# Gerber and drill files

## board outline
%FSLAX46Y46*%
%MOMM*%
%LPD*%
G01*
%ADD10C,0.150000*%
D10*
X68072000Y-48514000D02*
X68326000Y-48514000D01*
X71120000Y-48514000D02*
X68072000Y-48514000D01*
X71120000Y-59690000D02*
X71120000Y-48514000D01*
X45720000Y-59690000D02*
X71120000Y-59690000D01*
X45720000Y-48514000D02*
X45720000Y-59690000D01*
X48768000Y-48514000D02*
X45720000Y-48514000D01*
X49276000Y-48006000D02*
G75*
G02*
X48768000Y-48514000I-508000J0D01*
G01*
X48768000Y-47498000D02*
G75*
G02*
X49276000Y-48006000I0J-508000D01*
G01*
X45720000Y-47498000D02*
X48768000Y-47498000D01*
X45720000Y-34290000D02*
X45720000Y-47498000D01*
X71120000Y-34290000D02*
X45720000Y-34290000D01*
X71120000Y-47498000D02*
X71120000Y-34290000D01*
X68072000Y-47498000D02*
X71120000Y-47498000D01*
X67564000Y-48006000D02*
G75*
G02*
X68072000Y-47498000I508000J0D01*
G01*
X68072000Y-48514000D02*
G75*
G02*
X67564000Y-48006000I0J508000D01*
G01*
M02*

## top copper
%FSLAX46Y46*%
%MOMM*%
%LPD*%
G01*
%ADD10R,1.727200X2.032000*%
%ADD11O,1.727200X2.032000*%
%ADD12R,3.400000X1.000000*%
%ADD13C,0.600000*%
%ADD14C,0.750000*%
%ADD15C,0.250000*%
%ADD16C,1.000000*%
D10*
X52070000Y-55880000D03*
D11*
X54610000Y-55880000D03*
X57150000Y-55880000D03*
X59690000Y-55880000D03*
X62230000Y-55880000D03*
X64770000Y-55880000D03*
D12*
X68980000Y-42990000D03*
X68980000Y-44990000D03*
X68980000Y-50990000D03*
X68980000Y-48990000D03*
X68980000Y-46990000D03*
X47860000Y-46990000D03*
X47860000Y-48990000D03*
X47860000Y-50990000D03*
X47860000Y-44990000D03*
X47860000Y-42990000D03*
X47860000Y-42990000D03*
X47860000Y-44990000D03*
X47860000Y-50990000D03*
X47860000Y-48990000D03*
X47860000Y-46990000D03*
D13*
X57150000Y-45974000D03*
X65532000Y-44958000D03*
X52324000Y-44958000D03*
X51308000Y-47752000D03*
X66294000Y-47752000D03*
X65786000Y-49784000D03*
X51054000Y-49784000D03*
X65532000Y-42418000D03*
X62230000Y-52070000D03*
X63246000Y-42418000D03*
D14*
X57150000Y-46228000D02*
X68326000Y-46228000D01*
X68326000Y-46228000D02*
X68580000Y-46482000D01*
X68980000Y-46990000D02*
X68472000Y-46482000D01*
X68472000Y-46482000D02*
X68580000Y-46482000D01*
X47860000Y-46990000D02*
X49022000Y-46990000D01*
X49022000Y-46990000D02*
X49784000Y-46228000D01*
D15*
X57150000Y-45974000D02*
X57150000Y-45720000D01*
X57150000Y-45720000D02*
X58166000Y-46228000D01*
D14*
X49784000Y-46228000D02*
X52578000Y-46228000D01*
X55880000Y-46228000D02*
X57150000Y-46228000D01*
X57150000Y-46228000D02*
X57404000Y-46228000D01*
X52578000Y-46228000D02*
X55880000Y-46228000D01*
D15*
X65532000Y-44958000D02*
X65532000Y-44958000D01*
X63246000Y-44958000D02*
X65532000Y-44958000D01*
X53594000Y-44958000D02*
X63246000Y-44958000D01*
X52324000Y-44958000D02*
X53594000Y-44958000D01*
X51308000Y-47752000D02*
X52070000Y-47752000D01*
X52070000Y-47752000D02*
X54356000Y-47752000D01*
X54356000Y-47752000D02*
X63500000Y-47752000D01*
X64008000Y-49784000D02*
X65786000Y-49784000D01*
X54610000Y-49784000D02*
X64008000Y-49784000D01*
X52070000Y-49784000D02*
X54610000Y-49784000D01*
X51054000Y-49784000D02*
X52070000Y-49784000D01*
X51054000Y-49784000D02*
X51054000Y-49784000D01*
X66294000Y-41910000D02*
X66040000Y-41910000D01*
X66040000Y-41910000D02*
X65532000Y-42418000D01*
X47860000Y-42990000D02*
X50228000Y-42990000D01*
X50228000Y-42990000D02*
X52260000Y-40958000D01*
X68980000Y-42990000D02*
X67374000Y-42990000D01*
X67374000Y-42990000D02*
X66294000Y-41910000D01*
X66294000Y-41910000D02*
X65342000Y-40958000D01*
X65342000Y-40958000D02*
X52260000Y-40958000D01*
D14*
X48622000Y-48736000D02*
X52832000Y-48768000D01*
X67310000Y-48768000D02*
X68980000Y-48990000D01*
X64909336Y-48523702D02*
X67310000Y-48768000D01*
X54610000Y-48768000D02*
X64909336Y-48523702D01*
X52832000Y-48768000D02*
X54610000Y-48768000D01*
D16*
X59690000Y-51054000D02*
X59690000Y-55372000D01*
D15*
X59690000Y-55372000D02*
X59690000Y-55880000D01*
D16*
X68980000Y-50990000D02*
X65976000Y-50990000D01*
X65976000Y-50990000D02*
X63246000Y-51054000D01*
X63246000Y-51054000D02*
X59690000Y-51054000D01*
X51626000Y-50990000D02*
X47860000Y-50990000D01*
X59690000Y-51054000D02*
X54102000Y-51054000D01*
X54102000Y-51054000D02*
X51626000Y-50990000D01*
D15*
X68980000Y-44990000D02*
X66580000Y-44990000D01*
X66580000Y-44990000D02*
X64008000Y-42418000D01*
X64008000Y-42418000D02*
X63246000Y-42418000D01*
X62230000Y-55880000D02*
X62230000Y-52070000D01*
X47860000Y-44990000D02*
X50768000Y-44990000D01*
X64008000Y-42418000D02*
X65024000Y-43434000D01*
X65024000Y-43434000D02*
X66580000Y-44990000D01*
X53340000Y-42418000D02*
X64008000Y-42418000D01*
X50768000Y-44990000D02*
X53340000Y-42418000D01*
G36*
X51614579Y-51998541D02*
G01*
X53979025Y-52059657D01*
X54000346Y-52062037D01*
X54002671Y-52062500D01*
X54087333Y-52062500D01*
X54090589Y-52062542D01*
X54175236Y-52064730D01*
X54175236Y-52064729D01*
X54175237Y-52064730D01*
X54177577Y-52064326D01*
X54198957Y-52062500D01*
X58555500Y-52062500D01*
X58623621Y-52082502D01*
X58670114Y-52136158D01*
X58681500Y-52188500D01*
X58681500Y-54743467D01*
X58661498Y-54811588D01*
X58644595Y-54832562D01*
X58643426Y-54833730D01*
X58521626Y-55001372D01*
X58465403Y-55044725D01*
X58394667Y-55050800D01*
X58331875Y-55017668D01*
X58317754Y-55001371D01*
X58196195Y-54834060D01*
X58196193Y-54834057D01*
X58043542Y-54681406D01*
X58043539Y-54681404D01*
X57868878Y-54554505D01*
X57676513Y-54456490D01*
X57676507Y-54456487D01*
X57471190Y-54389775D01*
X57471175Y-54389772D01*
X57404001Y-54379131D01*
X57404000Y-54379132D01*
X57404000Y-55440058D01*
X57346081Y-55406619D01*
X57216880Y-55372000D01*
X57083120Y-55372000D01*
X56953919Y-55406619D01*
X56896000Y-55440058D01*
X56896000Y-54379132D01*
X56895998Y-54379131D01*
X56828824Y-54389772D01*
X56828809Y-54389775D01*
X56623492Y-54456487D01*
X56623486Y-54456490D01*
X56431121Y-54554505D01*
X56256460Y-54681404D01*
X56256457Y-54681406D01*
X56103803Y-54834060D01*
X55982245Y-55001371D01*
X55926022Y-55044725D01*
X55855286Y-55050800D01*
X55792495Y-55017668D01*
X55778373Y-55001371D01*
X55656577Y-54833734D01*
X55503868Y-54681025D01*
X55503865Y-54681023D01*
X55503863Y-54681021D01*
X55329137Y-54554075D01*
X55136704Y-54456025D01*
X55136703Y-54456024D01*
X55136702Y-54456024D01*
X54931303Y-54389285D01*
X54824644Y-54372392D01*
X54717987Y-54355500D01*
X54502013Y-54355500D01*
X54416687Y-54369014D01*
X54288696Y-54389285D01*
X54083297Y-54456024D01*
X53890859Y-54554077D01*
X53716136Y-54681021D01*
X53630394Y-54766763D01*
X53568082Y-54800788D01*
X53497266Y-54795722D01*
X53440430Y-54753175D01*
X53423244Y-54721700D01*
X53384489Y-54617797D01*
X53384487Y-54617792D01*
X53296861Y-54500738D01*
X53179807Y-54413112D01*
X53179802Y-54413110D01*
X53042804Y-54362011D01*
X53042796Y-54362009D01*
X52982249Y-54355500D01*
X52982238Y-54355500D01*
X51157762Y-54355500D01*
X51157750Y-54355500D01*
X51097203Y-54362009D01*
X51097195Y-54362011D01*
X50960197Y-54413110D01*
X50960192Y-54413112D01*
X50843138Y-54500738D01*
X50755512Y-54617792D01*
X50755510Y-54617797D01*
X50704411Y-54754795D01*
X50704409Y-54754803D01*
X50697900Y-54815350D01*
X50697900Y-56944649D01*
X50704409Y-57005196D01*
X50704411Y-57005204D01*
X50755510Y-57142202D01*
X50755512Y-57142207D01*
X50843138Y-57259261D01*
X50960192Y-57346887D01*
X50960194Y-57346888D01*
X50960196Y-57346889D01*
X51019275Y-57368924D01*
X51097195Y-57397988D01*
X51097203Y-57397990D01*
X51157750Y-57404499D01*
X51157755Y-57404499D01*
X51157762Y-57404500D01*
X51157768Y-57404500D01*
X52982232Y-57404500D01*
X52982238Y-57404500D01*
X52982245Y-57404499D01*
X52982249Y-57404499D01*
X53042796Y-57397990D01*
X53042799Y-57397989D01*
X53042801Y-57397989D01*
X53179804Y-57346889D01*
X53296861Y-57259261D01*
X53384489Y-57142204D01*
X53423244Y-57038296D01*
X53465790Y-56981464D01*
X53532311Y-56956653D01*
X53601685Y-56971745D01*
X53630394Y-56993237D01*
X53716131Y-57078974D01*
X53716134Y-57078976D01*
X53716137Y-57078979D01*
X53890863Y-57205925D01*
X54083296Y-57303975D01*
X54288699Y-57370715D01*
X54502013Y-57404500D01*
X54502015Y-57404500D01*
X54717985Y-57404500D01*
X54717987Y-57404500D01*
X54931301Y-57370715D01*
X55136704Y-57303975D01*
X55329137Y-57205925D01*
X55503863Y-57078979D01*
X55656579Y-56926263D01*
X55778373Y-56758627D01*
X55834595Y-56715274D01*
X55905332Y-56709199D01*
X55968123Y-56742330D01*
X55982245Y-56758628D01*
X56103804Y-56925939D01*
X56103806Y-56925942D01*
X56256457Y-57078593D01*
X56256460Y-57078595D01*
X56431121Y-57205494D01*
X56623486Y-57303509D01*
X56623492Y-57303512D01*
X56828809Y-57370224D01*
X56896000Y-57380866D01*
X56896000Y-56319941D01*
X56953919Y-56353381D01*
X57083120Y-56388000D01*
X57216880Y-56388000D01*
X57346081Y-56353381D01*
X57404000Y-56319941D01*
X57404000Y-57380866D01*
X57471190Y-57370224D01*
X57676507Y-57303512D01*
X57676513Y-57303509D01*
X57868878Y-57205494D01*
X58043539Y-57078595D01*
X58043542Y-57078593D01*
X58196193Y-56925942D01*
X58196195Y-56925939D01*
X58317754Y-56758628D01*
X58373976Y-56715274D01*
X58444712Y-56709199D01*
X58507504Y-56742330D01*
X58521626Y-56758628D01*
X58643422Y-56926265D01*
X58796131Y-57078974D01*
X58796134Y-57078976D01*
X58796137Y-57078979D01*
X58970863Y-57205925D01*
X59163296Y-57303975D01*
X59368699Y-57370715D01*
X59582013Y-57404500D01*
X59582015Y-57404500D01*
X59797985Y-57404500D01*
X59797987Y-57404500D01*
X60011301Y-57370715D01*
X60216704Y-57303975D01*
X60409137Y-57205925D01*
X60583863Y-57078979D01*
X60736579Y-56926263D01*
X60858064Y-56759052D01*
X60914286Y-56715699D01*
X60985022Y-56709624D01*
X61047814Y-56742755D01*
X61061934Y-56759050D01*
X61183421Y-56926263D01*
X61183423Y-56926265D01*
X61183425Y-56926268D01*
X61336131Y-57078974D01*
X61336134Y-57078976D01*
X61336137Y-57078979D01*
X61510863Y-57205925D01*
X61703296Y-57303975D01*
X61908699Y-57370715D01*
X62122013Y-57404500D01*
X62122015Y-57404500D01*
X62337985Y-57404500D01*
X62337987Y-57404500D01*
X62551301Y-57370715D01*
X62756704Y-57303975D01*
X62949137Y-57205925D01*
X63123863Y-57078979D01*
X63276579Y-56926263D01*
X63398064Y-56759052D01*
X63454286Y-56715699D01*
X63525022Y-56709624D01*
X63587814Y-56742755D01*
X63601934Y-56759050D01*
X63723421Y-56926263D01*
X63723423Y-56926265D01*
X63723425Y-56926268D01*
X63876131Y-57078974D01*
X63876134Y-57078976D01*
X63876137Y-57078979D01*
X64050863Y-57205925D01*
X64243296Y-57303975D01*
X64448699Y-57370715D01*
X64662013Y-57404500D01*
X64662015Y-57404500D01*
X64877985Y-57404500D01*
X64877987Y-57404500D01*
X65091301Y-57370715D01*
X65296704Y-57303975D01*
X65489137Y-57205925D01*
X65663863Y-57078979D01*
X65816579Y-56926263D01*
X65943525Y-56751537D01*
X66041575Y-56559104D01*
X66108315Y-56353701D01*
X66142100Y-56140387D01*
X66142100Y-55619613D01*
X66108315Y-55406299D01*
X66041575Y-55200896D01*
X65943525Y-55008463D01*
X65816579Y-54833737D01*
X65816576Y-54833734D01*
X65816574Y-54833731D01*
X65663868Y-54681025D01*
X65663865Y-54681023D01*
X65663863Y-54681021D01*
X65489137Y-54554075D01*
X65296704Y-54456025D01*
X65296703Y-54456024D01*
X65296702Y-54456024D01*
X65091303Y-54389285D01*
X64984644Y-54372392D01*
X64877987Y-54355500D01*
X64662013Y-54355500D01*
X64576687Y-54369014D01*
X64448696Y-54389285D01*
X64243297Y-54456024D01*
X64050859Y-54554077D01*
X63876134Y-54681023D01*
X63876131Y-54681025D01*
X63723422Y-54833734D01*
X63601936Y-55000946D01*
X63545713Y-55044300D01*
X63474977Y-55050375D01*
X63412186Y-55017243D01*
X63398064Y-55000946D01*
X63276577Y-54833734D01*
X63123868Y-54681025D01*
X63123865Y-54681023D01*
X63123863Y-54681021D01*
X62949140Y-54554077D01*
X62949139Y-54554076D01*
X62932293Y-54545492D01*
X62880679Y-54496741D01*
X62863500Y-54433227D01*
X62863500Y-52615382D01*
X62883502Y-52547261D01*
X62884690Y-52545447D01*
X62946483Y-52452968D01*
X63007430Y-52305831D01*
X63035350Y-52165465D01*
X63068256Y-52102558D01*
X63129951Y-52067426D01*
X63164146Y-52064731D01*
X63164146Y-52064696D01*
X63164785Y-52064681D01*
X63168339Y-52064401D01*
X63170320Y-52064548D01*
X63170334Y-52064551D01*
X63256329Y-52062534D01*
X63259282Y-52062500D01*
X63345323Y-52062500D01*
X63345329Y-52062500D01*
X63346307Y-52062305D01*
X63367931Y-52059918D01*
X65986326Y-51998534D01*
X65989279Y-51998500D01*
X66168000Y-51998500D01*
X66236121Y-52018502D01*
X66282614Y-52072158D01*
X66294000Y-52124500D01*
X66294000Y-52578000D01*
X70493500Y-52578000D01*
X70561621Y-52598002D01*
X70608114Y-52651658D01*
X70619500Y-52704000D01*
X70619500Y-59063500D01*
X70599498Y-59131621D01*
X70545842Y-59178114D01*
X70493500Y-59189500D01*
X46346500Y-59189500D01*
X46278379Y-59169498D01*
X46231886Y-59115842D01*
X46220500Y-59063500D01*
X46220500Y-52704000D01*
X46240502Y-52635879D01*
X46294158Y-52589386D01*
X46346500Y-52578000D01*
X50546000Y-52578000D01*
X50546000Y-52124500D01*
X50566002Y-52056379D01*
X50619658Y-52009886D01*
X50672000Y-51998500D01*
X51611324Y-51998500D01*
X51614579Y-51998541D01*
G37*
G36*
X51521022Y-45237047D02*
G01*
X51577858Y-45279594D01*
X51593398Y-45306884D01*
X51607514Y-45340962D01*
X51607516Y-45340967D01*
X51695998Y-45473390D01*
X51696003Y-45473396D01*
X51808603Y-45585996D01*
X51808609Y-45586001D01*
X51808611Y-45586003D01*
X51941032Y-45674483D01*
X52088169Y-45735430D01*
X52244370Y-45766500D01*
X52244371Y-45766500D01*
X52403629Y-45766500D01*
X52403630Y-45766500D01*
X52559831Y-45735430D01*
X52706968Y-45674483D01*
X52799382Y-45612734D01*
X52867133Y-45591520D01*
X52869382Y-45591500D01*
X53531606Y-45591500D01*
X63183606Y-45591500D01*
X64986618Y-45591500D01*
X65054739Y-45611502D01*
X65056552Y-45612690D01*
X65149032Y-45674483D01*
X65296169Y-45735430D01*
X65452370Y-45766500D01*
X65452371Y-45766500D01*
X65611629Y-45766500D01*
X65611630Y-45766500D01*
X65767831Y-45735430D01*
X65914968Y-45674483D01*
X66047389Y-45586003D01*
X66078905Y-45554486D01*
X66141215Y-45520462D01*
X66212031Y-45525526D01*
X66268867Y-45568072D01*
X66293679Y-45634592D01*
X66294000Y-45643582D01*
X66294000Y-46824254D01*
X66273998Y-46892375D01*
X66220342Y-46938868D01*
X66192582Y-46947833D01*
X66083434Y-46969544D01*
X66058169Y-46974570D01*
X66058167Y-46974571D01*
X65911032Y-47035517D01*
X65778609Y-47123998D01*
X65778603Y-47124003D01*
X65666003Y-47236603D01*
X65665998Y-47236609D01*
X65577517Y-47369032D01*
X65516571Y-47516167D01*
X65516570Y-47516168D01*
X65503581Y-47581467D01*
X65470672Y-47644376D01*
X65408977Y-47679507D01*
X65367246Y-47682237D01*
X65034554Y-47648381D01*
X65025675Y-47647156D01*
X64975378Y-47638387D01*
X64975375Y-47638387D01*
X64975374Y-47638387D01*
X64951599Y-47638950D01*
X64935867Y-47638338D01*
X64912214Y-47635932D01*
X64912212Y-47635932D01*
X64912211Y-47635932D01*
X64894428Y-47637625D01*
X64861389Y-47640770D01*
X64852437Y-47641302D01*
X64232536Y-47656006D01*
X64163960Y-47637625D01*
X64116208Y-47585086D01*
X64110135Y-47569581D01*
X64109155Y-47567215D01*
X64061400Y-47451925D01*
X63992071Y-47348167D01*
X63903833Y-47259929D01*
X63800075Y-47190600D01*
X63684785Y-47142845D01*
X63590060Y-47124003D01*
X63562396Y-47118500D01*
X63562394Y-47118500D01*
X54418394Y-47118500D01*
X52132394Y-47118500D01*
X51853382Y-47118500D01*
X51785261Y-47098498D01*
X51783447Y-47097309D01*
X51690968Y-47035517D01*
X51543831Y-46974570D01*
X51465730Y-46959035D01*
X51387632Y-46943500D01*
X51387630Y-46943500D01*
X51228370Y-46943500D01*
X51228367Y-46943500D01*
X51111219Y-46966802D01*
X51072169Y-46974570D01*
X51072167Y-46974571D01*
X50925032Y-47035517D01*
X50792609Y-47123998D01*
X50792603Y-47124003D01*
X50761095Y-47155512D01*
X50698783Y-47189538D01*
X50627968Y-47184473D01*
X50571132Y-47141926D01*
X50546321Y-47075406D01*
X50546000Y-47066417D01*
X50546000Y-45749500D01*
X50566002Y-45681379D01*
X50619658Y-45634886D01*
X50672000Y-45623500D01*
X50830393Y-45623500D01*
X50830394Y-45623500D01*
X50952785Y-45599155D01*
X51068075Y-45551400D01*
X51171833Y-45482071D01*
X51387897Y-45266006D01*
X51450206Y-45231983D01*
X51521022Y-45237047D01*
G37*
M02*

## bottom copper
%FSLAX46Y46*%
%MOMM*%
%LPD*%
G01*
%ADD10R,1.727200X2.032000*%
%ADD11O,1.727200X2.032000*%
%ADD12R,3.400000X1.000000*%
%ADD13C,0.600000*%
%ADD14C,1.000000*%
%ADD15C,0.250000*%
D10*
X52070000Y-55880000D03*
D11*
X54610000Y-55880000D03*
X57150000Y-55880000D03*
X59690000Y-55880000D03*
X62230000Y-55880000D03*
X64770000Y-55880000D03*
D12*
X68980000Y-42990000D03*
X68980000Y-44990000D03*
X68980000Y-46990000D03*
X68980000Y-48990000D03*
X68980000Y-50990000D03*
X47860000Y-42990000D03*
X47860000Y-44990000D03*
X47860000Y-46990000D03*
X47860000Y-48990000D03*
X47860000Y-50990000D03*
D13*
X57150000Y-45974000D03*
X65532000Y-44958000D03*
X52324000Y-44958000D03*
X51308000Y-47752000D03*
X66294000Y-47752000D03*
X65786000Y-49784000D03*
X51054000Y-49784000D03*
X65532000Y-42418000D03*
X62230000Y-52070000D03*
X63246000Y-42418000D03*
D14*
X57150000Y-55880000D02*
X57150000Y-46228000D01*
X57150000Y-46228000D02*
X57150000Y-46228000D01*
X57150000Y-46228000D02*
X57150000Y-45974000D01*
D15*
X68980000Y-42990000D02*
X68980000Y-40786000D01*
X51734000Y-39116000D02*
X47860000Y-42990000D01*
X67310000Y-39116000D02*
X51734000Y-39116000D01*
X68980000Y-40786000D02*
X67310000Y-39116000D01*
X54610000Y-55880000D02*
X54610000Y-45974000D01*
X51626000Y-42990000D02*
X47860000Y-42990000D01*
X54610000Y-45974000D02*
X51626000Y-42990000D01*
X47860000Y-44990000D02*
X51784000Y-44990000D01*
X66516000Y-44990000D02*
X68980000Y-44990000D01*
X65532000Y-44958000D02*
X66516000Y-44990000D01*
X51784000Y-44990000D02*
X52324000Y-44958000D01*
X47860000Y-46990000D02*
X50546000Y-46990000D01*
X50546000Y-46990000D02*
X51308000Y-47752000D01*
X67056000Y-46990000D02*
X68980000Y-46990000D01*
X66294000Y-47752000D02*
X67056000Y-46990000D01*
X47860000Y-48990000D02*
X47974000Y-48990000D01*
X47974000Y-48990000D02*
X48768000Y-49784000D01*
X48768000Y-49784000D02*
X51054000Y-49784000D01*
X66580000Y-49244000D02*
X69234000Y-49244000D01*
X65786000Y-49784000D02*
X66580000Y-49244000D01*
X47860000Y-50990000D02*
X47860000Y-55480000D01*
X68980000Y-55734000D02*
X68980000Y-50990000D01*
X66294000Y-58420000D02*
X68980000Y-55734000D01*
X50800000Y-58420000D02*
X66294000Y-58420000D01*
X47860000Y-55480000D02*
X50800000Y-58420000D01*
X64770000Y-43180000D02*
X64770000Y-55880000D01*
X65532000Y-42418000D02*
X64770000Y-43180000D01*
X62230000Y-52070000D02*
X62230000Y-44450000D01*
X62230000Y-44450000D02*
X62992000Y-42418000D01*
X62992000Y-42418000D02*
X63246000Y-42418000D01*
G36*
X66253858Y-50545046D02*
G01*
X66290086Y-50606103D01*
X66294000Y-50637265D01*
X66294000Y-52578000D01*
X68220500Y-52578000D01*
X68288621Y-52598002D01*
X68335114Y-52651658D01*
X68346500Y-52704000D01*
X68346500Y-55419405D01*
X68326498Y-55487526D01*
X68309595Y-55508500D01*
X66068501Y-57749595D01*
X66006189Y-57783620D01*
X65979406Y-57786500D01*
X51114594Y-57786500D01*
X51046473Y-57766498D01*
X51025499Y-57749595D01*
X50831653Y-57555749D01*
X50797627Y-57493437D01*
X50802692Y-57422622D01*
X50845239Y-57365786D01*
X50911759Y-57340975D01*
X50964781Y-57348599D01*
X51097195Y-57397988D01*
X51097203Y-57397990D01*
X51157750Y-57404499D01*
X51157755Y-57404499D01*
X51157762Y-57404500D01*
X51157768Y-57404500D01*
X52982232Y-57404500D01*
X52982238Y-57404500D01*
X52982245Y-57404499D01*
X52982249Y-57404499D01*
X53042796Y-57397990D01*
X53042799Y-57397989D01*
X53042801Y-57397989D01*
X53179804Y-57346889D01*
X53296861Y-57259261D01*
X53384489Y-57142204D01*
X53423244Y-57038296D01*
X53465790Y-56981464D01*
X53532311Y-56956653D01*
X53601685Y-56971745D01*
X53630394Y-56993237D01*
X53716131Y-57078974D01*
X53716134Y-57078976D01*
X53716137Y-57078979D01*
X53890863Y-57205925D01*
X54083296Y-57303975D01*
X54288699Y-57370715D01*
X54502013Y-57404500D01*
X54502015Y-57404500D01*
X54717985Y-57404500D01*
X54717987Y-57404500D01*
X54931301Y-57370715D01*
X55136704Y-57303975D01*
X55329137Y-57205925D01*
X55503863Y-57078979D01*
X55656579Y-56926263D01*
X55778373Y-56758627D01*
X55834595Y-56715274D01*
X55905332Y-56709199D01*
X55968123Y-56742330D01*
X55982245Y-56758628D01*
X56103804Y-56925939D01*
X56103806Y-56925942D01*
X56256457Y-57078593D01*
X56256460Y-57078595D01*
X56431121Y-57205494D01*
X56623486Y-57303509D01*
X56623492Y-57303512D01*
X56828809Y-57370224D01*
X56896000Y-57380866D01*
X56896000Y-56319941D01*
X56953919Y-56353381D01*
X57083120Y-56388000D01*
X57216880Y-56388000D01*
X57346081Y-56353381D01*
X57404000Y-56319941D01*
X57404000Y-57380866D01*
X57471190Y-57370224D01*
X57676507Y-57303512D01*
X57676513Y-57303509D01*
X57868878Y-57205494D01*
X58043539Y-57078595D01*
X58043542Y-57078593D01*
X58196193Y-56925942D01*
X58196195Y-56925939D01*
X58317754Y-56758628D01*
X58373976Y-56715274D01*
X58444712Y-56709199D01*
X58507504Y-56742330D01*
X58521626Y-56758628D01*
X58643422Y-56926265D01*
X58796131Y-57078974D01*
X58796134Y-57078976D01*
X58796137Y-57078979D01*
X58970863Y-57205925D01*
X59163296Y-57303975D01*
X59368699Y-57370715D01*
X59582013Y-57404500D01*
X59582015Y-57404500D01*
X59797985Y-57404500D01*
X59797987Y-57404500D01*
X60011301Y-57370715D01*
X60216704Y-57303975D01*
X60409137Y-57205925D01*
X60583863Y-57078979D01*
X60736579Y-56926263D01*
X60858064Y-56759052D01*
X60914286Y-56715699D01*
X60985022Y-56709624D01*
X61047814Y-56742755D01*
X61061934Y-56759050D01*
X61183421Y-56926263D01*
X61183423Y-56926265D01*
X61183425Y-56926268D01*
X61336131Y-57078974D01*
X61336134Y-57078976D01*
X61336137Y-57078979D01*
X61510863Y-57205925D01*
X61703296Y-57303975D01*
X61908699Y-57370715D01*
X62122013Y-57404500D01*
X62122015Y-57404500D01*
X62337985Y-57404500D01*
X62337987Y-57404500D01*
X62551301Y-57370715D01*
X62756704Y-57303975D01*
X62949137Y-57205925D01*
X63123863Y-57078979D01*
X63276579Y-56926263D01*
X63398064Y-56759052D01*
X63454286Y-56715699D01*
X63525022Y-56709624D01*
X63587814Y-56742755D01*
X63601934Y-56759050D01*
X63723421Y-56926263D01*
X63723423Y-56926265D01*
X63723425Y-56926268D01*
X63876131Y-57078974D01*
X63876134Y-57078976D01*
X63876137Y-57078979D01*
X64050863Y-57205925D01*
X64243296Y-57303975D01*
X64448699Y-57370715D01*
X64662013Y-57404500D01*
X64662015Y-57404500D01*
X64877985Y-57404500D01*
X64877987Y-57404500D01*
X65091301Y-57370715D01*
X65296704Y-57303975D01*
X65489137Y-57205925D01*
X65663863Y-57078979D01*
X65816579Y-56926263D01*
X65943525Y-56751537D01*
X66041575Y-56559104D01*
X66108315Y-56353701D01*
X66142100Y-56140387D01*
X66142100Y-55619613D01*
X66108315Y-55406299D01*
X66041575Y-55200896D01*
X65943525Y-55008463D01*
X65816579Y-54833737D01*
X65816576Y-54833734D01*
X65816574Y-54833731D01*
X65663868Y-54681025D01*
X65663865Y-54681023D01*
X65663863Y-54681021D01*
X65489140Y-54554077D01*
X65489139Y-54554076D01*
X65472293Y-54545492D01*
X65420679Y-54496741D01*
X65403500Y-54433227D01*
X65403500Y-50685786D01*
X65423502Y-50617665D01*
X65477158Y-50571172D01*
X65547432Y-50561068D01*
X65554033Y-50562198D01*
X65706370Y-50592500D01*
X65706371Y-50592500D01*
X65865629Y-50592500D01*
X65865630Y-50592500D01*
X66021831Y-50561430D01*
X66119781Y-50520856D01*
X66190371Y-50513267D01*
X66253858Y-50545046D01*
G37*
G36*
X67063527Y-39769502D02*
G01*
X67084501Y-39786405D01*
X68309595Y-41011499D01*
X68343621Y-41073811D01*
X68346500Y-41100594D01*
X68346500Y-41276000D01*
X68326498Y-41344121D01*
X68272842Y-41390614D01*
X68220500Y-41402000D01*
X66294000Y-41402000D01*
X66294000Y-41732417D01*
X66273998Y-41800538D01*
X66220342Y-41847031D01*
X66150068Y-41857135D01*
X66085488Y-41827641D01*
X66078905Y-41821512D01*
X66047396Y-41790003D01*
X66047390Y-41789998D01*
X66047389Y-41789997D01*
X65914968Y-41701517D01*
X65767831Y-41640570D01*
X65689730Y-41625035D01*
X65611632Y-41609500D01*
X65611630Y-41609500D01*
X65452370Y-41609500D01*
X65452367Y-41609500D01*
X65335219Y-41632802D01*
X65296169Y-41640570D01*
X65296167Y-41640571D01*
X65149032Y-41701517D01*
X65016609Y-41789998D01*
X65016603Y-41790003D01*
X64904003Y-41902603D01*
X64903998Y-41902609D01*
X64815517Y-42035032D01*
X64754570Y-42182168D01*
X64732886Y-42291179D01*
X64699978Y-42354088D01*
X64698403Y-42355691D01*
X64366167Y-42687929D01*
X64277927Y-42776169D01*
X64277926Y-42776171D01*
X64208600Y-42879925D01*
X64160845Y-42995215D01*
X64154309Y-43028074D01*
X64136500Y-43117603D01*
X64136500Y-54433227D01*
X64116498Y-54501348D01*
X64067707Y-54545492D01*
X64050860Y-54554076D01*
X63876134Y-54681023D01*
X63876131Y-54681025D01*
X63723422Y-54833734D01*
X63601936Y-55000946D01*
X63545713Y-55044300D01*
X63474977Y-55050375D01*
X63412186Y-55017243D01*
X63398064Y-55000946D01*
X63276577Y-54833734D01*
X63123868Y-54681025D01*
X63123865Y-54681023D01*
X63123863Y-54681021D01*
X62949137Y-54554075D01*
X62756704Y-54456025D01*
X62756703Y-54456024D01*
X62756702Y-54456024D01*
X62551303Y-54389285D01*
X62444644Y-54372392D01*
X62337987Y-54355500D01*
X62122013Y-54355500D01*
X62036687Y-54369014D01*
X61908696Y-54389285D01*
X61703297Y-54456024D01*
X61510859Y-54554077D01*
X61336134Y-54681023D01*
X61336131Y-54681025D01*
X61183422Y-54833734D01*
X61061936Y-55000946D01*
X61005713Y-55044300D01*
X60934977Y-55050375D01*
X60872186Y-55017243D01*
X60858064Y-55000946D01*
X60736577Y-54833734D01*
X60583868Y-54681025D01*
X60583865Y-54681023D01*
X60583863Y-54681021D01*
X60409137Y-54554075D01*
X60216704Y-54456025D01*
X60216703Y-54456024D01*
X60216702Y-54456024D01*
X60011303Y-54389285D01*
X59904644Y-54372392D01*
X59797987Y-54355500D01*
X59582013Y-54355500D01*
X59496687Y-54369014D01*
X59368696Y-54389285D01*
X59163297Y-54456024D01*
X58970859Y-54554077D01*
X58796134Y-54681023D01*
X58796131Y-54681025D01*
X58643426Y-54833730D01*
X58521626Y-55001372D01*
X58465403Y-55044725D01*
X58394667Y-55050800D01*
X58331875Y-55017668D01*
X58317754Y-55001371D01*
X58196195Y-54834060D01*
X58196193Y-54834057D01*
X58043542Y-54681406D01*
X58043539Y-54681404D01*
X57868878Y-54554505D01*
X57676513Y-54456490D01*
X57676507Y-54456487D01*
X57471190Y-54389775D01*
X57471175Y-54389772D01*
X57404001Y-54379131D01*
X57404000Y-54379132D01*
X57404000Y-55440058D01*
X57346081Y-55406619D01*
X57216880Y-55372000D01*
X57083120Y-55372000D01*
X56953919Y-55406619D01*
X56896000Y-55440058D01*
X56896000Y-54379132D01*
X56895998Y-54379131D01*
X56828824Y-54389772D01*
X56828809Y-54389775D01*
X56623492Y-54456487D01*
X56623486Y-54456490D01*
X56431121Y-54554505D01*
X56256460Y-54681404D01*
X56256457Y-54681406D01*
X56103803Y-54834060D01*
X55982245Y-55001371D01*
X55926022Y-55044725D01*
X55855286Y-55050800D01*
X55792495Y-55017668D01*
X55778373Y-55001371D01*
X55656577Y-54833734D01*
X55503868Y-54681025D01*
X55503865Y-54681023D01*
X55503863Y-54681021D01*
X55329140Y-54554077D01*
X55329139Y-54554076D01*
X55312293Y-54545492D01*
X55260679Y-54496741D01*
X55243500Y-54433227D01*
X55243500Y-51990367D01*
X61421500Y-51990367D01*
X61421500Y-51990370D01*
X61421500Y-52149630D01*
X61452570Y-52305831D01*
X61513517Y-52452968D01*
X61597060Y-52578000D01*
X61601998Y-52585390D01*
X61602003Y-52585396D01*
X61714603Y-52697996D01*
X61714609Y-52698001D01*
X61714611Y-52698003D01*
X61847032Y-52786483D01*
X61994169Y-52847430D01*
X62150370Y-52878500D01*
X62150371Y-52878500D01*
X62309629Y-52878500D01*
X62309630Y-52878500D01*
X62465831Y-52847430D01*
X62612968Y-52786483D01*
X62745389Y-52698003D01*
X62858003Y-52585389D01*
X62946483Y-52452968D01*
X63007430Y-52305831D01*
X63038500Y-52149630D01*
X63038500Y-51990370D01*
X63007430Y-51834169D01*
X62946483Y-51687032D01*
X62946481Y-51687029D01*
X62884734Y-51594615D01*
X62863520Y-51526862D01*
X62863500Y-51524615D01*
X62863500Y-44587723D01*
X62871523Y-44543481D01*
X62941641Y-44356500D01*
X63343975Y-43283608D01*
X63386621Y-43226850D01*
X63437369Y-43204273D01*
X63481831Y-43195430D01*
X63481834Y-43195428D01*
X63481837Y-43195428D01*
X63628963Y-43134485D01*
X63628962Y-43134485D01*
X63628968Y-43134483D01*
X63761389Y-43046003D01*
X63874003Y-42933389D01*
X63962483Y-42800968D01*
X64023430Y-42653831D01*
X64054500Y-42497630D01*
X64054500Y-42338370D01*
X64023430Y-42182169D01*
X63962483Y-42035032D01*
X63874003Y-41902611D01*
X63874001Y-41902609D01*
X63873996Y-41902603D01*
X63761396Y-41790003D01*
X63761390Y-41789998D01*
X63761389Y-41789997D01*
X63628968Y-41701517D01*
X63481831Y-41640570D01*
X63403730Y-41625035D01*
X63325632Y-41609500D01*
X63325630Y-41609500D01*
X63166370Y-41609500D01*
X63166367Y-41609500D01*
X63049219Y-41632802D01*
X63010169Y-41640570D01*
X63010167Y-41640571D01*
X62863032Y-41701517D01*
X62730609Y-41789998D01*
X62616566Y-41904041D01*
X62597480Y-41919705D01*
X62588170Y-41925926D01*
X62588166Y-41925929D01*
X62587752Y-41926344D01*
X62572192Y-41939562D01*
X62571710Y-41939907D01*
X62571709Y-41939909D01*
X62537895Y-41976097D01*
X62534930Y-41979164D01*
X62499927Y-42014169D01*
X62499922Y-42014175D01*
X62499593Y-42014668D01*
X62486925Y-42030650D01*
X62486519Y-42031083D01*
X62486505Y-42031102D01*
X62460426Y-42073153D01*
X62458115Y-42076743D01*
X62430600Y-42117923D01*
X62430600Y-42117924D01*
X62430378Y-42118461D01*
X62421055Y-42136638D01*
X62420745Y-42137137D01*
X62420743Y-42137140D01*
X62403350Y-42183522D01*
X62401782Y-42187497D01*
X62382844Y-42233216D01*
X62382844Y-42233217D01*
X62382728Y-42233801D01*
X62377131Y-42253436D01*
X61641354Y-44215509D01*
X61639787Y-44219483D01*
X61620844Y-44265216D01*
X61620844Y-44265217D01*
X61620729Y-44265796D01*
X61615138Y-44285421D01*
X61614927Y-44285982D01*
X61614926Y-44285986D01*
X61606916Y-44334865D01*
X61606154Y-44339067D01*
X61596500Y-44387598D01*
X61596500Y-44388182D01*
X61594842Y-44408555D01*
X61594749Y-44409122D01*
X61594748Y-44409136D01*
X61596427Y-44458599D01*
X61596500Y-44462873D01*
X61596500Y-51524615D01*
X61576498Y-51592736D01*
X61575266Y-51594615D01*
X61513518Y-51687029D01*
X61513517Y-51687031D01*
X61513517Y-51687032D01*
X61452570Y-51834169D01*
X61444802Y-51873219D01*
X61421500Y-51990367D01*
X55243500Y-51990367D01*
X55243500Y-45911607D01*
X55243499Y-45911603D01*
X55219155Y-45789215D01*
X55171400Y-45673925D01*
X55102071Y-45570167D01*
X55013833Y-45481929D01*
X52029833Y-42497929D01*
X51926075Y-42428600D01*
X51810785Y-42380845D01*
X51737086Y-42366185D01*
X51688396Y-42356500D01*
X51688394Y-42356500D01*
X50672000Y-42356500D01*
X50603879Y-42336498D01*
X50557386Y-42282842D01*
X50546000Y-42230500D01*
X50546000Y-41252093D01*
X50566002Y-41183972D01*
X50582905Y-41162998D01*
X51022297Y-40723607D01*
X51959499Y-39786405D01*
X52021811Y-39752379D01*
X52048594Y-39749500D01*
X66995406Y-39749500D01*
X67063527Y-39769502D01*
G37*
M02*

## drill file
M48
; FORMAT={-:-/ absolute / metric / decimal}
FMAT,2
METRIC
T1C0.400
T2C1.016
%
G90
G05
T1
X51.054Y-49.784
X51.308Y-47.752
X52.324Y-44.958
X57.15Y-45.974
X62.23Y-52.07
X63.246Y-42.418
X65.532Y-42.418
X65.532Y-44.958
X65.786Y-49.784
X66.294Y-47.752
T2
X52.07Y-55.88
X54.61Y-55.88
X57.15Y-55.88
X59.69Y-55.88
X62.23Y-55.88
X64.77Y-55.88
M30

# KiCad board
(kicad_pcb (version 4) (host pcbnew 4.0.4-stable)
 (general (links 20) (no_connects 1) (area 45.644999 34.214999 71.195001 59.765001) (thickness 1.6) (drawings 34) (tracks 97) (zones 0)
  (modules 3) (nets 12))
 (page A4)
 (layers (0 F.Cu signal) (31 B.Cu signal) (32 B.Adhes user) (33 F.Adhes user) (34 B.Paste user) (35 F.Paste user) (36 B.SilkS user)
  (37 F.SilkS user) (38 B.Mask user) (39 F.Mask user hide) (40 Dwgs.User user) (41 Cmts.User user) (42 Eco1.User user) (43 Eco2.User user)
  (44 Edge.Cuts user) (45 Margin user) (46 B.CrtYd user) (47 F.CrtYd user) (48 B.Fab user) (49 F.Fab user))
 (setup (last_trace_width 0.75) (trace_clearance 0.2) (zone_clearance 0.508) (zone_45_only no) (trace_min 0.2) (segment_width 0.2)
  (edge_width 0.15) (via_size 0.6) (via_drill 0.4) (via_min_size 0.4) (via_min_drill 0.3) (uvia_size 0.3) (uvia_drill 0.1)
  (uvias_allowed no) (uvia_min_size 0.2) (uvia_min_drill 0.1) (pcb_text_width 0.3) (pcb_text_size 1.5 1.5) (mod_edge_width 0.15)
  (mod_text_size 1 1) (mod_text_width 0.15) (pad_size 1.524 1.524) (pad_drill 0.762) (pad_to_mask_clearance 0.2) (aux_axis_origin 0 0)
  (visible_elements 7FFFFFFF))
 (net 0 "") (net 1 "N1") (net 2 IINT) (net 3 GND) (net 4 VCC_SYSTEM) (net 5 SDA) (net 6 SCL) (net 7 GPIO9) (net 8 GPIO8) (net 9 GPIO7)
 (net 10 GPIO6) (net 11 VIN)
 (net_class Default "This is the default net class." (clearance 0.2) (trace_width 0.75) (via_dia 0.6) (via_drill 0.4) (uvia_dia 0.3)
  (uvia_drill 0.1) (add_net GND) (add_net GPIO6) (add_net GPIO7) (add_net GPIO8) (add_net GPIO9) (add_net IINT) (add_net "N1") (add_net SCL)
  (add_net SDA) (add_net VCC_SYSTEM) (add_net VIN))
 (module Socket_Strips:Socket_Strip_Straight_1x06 (layer F.Cu) (at 52.07 55.88)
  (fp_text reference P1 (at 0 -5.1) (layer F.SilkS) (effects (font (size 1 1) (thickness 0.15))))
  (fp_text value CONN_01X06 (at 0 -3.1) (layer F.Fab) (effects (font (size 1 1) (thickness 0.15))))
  (pad 1 thru_hole rect (at 0 0) (size 1.7272 2.032) (drill 1.016) (layers *.Cu *.Mask F.SilkS) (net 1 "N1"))
  (pad 2 thru_hole oval (at 2.54 0) (size 1.7272 2.032) (drill 1.016) (layers *.Cu *.Mask F.SilkS) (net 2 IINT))
  (pad 3 thru_hole oval (at 5.08 0) (size 1.7272 2.032) (drill 1.016) (layers *.Cu *.Mask F.SilkS) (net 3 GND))
  (pad 4 thru_hole oval (at 7.62 0) (size 1.7272 2.032) (drill 1.016) (layers *.Cu *.Mask F.SilkS) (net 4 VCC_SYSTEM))
  (pad 5 thru_hole oval (at 10.16 0) (size 1.7272 2.032) (drill 1.016) (layers *.Cu *.Mask F.SilkS) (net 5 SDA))
  (pad 6 thru_hole oval (at 12.7 0) (size 1.7272 2.032) (drill 1.016) (layers *.Cu *.Mask F.SilkS) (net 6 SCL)))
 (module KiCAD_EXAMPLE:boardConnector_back (layer F.Cu) (at 68.58 46.99 270)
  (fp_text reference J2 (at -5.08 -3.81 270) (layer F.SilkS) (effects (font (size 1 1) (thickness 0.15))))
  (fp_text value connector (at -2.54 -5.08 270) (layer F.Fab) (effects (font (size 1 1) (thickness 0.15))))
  (pad 10 smd rect (at -4 -0.4 270) (size 1 3.4) (layers B.Cu B.Paste B.Mask) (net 2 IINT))
  (pad 9 smd rect (at -2 -0.4 270) (size 1 3.4) (layers B.Cu B.Paste B.Mask) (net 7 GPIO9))
  (pad 8 smd rect (at 0 -0.4 270) (size 1 3.4) (layers B.Cu B.Paste B.Mask) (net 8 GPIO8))
  (pad 7 smd rect (at 2 -0.4 270) (size 1 3.4) (layers B.Cu B.Paste B.Mask) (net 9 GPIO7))
  (pad 6 smd rect (at 4 -0.4 270) (size 1 3.4) (layers B.Cu B.Paste B.Mask) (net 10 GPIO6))
  (pad 5 smd rect (at -4 -0.4 270) (size 1 3.4) (layers F.Cu F.Paste F.Mask) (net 6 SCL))
  (pad 4 smd rect (at -2 -0.4 270) (size 1 3.4) (layers F.Cu F.Paste F.Mask) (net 5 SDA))
  (pad 1 smd rect (at 4 -0.4 270) (size 1 3.4) (layers F.Cu F.Paste F.Mask) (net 4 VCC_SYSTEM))
  (pad 2 smd rect (at 2 -0.4 270) (size 1 3.4) (layers F.Cu F.Paste F.Mask) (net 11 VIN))
  (pad 3 smd rect (at 0 -0.4 270) (size 1 3.4) (layers F.Cu F.Paste F.Mask) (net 3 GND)))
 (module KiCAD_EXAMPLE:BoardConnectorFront (layer F.Cu) (at 48.26 46.99 270)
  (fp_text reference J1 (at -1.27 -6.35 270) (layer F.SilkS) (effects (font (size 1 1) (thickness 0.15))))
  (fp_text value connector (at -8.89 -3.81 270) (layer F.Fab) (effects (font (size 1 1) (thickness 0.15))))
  (pad 10 smd rect (at -4 0.4 270) (size 1 3.4) (layers B.Cu B.Paste B.Mask) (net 2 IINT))
  (pad 9 smd rect (at -2 0.4 270) (size 1 3.4) (layers B.Cu B.Paste B.Mask) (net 7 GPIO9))
  (pad 8 smd rect (at 0 0.4 270) (size 1 3.4) (layers B.Cu B.Paste B.Mask) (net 8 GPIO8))
  (pad 7 smd rect (at 2 0.4 270) (size 1 3.4) (layers B.Cu B.Paste B.Mask) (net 9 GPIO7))
  (pad 6 smd rect (at 4 0.4 270) (size 1 3.4) (layers B.Cu B.Paste B.Mask) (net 10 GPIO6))
  (pad 3 smd rect (at 0 0.4 270) (size 1 3.4) (layers F.Cu F.Paste F.Mask) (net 3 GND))
  (pad 2 smd rect (at 2 0.4 270) (size 1 3.4) (layers F.Cu F.Paste F.Mask) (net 11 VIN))
  (pad 1 smd rect (at 4 0.4 270) (size 1 3.4) (layers F.Cu F.Paste F.Mask) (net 4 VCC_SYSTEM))
  (pad 4 smd rect (at -2 0.4 270) (size 1 3.4) (layers F.Cu F.Paste F.Mask) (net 5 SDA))
  (pad 5 smd rect (at -4 0.4 270) (size 1 3.4) (layers F.Cu F.Paste F.Mask) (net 6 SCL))
  (pad 5 smd rect (at -4 0.4 270) (size 1 3.4) (layers F.Cu F.Paste F.Mask) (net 6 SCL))
  (pad 4 smd rect (at -2 0.4 270) (size 1 3.4) (layers F.Cu F.Paste F.Mask) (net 5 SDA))
  (pad 1 smd rect (at 4 0.4 270) (size 1 3.4) (layers F.Cu F.Paste F.Mask) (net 4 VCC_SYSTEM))
  (pad 2 smd rect (at 2 0.4 270) (size 1 3.4) (layers F.Cu F.Paste F.Mask) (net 11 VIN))
  (pad 3 smd rect (at 0 0.4 270) (size 1 3.4) (layers F.Cu F.Paste F.Mask) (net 3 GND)))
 (gr_line (start 68.072 48.514) (end 68.326 48.514) (angle 90) (layer Edge.Cuts) (width 0.15))
 (gr_line (start 71.12 48.514) (end 68.072 48.514) (angle 90) (layer Edge.Cuts) (width 0.15))
 (gr_line (start 71.12 59.69) (end 71.12 48.514) (angle 90) (layer Edge.Cuts) (width 0.15))
 (gr_line (start 45.72 59.69) (end 71.12 59.69) (angle 90) (layer Edge.Cuts) (width 0.15))
 (gr_line (start 45.72 48.514) (end 45.72 59.69) (angle 90) (layer Edge.Cuts) (width 0.15))
 (gr_line (start 48.768 48.514) (end 45.72 48.514) (angle 90) (layer Edge.Cuts) (width 0.15))
 (gr_arc (start 48.768 48.006) (end 49.276 48.006) (angle 90) (layer Edge.Cuts) (width 0.15))
 (gr_arc (start 48.768 48.006) (end 48.768 47.498) (angle 90) (layer Edge.Cuts) (width 0.15))
 (gr_line (start 45.72 47.498) (end 48.768 47.498) (angle 90) (layer Edge.Cuts) (width 0.15))
 (gr_line (start 45.72 34.29) (end 45.72 47.498) (angle 90) (layer Edge.Cuts) (width 0.15))
 (gr_line (start 71.12 34.29) (end 45.72 34.29) (angle 90) (layer Edge.Cuts) (width 0.15))
 (gr_line (start 71.12 47.498) (end 71.12 34.29) (angle 90) (layer Edge.Cuts) (width 0.15))
 (gr_line (start 68.072 47.498) (end 71.12 47.498) (angle 90) (layer Edge.Cuts) (width 0.15))
 (gr_arc (start 68.072 48.006) (end 67.564 48.006) (angle 90) (layer Edge.Cuts) (width 0.15))
 (gr_arc (start 68.072 48.006) (end 68.072 48.514) (angle 90) (layer Edge.Cuts) (width 0.15))
 (segment (start 57.15 46.228) (end 68.326 46.228) (width 0.75) (layer F.Cu) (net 3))
 (segment (start 68.326 46.228) (end 68.58 46.482) (width 0.75) (layer F.Cu) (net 3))
 (segment (start 68.98 46.99) (end 68.472 46.482) (width 0.75) (layer F.Cu) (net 3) (status 400000))
 (segment (start 68.472 46.482) (end 68.58 46.482) (width 0.75) (layer F.Cu) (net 3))
 (segment (start 47.86 46.99) (end 49.022 46.99) (width 0.75) (layer F.Cu) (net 3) (status C00000))
 (segment (start 49.022 46.99) (end 49.784 46.228) (width 0.75) (layer F.Cu) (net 3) (status 400000))
 (segment (start 57.15 55.88) (end 57.15 46.228) (width 1) (layer B.Cu) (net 3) (status 400000))
 (segment (start 57.15 46.228) (end 57.15 46.228) (width 1) (layer B.Cu) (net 3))
 (segment (start 57.15 46.228) (end 57.15 45.974) (width 1) (layer B.Cu) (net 3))
 (via (at 57.15 45.974) (size 0.6) (drill 0.4) (layers F.Cu B.Cu) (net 3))
 (segment (start 57.15 45.974) (end 57.15 45.72) (width 0.25) (layer F.Cu) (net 3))
 (segment (start 57.15 45.72) (end 58.166 46.228) (width 0.25) (layer F.Cu) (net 3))
 (segment (start 49.784 46.228) (end 52.578 46.228) (width 0.75) (layer F.Cu) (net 3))
 (segment (start 55.88 46.228) (end 57.15 46.228) (width 0.75) (layer F.Cu) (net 3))
 (segment (start 57.15 46.228) (end 57.404 46.228) (width 0.75) (layer F.Cu) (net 3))
 (segment (start 52.578 46.228) (end 55.88 46.228) (width 0.75) (layer F.Cu) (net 3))
 (segment (start 68.98 42.99) (end 68.98 40.786) (width 0.25) (layer B.Cu) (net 2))
 (segment (start 51.734 39.116) (end 47.86 42.99) (width 0.25) (layer B.Cu) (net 2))
 (segment (start 67.31 39.116) (end 51.734 39.116) (width 0.25) (layer B.Cu) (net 2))
 (segment (start 68.98 40.786) (end 67.31 39.116) (width 0.25) (layer B.Cu) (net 2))
 (segment (start 54.61 55.88) (end 54.61 45.974) (width 0.25) (layer B.Cu) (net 2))
 (segment (start 51.626 42.99) (end 47.86 42.99) (width 0.25) (layer B.Cu) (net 2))
 (segment (start 54.61 45.974) (end 51.626 42.99) (width 0.25) (layer B.Cu) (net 2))
 (segment (start 47.86 44.99) (end 51.784 44.99) (width 0.25) (layer B.Cu) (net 7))
 (segment (start 66.516 44.99) (end 68.98 44.99) (width 0.25) (layer B.Cu) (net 7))
 (segment (start 65.532 44.958) (end 66.516 44.99) (width 0.25) (layer B.Cu) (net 7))
 (via (at 65.532 44.958) (size 0.6) (drill 0.4) (layers F.Cu B.Cu) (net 7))
 (segment (start 65.532 44.958) (end 65.532 44.958) (width 0.25) (layer F.Cu) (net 7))
 (segment (start 63.246 44.958) (end 65.532 44.958) (width 0.25) (layer F.Cu) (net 7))
 (segment (start 53.594 44.958) (end 63.246 44.958) (width 0.25) (layer F.Cu) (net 7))
 (segment (start 52.324 44.958) (end 53.594 44.958) (width 0.25) (layer F.Cu) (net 7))
 (via (at 52.324 44.958) (size 0.6) (drill 0.4) (layers F.Cu B.Cu) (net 7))
 (segment (start 51.784 44.99) (end 52.324 44.958) (width 0.25) (layer B.Cu) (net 7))
 (segment (start 47.86 46.99) (end 50.546 46.99) (width 0.25) (layer B.Cu) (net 8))
 (segment (start 50.546 46.99) (end 51.308 47.752) (width 0.25) (layer B.Cu) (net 8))
 (via (at 51.308 47.752) (size 0.6) (drill 0.4) (layers F.Cu B.Cu) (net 8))
 (segment (start 51.308 47.752) (end 52.07 47.752) (width 0.25) (layer F.Cu) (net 8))
 (segment (start 52.07 47.752) (end 54.356 47.752) (width 0.25) (layer F.Cu) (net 8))
 (segment (start 54.356 47.752) (end 63.5 47.752) (width 0.25) (layer F.Cu) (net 8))
 (segment (start 67.056 46.99) (end 68.98 46.99) (width 0.25) (layer B.Cu) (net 8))
 (segment (start 66.294 47.752) (end 67.056 46.99) (width 0.25) (layer B.Cu) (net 8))
 (via (at 66.294 47.752) (size 0.6) (drill 0.4) (layers F.Cu B.Cu) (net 8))
 (segment (start 47.86 48.99) (end 47.974 48.99) (width 0.25) (layer B.Cu) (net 9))
 (segment (start 47.974 48.99) (end 48.768 49.784) (width 0.25) (layer B.Cu) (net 9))
 (segment (start 48.768 49.784) (end 51.054 49.784) (width 0.25) (layer B.Cu) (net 9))
 (segment (start 66.58 49.244) (end 69.234 49.244) (width 0.25) (layer B.Cu) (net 9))
 (segment (start 65.786 49.784) (end 66.58 49.244) (width 0.25) (layer B.Cu) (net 9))
 (via (at 65.786 49.784) (size 0.6) (drill 0.4) (layers F.Cu B.Cu) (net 9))
 (segment (start 64.008 49.784) (end 65.786 49.784) (width 0.25) (layer F.Cu) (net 9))
 (segment (start 54.61 49.784) (end 64.008 49.784) (width 0.25) (layer F.Cu) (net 9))
 (segment (start 52.07 49.784) (end 54.61 49.784) (width 0.25) (layer F.Cu) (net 9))
 (segment (start 51.054 49.784) (end 52.07 49.784) (width 0.25) (layer F.Cu) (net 9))
 (segment (start 51.054 49.784) (end 51.054 49.784) (width 0.25) (layer F.Cu) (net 9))
 (via (at 51.054 49.784) (size 0.6) (drill 0.4) (layers F.Cu B.Cu) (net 9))
 (segment (start 47.86 50.99) (end 47.86 55.48) (width 0.25) (layer B.Cu) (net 10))
 (segment (start 68.98 55.734) (end 68.98 50.99) (width 0.25) (layer B.Cu) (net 10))
 (segment (start 66.294 58.42) (end 68.98 55.734) (width 0.25) (layer B.Cu) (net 10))
 (segment (start 50.8 58.42) (end 66.294 58.42) (width 0.25) (layer B.Cu) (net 10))
 (segment (start 47.86 55.48) (end 50.8 58.42) (width 0.25) (layer B.Cu) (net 10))
 (segment (start 66.294 41.91) (end 66.04 41.91) (width 0.25) (layer F.Cu) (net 6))
 (segment (start 64.77 43.18) (end 64.77 55.88) (width 0.25) (layer B.Cu) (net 6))
 (segment (start 65.532 42.418) (end 64.77 43.18) (width 0.25) (layer B.Cu) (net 6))
 (via (at 65.532 42.418) (size 0.6) (drill 0.4) (layers F.Cu B.Cu) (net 6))
 (segment (start 66.04 41.91) (end 65.532 42.418) (width 0.25) (layer F.Cu) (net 6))
 (segment (start 47.86 42.99) (end 50.228 42.99) (width 0.25) (layer F.Cu) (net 6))
 (segment (start 50.228 42.99) (end 52.26 40.958) (width 0.25) (layer F.Cu) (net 6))
 (segment (start 68.98 42.99) (end 67.374 42.99) (width 0.25) (layer F.Cu) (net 6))
 (segment (start 67.374 42.99) (end 66.294 41.91) (width 0.25) (layer F.Cu) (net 6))
 (segment (start 66.294 41.91) (end 65.342 40.958) (width 0.25) (layer F.Cu) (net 6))
 (segment (start 65.342 40.958) (end 52.26 40.958) (width 0.25) (layer F.Cu) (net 6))
 (segment (start 48.622 48.736) (end 52.832 48.768) (width 0.75) (layer F.Cu) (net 11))
 (segment (start 67.31 48.768) (end 68.98 48.99) (width 0.75) (layer F.Cu) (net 11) (status 800000))
 (segment (start 64.909336 48.523702) (end 67.31 48.768) (width 0.75) (layer F.Cu) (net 11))
 (segment (start 54.61 48.768) (end 64.909336 48.523702) (width 0.75) (layer F.Cu) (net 11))
 (segment (start 52.832 48.768) (end 54.61 48.768) (width 0.75) (layer F.Cu) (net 11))
 (segment (start 59.69 51.054) (end 59.69 55.372) (width 1) (layer F.Cu) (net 4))
 (segment (start 59.69 55.372) (end 59.69 55.88) (width 0.25) (layer F.Cu) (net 4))
 (segment (start 68.98 50.99) (end 65.976 50.99) (width 1) (layer F.Cu) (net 4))
 (segment (start 65.976 50.99) (end 63.246 51.054) (width 1) (layer F.Cu) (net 4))
 (segment (start 63.246 51.054) (end 59.69 51.054) (width 1) (layer F.Cu) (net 4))
 (segment (start 51.626 50.99) (end 47.86 50.99) (width 1) (layer F.Cu) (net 4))
 (segment (start 59.69 51.054) (end 54.102 51.054) (width 1) (layer F.Cu) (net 4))
 (segment (start 54.102 51.054) (end 51.626 50.99) (width 1) (layer F.Cu) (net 4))
 (segment (start 68.98 44.99) (end 66.58 44.99) (width 0.25) (layer F.Cu) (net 5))
 (segment (start 66.58 44.99) (end 64.008 42.418) (width 0.25) (layer F.Cu) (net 5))
 (segment (start 64.008 42.418) (end 63.246 42.418) (width 0.25) (layer F.Cu) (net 5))
 (segment (start 62.23 55.88) (end 62.23 52.07) (width 0.25) (layer F.Cu) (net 5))
 (segment (start 62.23 52.07) (end 62.23 44.45) (width 0.25) (layer B.Cu) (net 5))
 (via (at 62.23 52.07) (size 0.6) (drill 0.4) (layers F.Cu B.Cu) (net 5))
 (segment (start 62.23 44.45) (end 62.992 42.418) (width 0.25) (layer B.Cu) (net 5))
 (segment (start 62.992 42.418) (end 63.246 42.418) (width 0.25) (layer B.Cu) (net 5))
 (via (at 63.246 42.418) (size 0.6) (drill 0.4) (layers F.Cu B.Cu) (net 5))
 (segment (start 47.86 44.99) (end 50.768 44.99) (width 0.25) (layer F.Cu) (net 5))
 (segment (start 64.008 42.418) (end 65.024 43.434) (width 0.25) (layer F.Cu) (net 5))
 (segment (start 65.024 43.434) (end 66.58 44.99) (width 0.25) (layer F.Cu) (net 5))
 (segment (start 53.34 42.418) (end 64.008 42.418) (width 0.25) (layer F.Cu) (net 5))
 (segment (start 50.768 44.99) (end 53.34 42.418) (width 0.25) (layer F.Cu) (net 5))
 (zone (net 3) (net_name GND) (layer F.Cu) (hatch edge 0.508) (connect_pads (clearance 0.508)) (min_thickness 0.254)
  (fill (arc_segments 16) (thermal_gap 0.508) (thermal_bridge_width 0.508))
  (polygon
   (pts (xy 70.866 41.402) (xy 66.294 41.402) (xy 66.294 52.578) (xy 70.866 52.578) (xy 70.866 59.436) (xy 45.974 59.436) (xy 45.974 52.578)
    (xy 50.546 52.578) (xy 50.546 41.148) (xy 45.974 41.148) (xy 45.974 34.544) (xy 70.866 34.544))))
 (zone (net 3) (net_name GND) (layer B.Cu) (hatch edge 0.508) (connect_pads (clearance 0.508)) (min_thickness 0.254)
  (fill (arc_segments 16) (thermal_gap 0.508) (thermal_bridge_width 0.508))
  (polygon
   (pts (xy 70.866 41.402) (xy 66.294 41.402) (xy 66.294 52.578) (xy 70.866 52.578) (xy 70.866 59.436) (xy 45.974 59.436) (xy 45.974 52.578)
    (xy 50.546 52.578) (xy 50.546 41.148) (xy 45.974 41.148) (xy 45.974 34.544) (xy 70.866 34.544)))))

